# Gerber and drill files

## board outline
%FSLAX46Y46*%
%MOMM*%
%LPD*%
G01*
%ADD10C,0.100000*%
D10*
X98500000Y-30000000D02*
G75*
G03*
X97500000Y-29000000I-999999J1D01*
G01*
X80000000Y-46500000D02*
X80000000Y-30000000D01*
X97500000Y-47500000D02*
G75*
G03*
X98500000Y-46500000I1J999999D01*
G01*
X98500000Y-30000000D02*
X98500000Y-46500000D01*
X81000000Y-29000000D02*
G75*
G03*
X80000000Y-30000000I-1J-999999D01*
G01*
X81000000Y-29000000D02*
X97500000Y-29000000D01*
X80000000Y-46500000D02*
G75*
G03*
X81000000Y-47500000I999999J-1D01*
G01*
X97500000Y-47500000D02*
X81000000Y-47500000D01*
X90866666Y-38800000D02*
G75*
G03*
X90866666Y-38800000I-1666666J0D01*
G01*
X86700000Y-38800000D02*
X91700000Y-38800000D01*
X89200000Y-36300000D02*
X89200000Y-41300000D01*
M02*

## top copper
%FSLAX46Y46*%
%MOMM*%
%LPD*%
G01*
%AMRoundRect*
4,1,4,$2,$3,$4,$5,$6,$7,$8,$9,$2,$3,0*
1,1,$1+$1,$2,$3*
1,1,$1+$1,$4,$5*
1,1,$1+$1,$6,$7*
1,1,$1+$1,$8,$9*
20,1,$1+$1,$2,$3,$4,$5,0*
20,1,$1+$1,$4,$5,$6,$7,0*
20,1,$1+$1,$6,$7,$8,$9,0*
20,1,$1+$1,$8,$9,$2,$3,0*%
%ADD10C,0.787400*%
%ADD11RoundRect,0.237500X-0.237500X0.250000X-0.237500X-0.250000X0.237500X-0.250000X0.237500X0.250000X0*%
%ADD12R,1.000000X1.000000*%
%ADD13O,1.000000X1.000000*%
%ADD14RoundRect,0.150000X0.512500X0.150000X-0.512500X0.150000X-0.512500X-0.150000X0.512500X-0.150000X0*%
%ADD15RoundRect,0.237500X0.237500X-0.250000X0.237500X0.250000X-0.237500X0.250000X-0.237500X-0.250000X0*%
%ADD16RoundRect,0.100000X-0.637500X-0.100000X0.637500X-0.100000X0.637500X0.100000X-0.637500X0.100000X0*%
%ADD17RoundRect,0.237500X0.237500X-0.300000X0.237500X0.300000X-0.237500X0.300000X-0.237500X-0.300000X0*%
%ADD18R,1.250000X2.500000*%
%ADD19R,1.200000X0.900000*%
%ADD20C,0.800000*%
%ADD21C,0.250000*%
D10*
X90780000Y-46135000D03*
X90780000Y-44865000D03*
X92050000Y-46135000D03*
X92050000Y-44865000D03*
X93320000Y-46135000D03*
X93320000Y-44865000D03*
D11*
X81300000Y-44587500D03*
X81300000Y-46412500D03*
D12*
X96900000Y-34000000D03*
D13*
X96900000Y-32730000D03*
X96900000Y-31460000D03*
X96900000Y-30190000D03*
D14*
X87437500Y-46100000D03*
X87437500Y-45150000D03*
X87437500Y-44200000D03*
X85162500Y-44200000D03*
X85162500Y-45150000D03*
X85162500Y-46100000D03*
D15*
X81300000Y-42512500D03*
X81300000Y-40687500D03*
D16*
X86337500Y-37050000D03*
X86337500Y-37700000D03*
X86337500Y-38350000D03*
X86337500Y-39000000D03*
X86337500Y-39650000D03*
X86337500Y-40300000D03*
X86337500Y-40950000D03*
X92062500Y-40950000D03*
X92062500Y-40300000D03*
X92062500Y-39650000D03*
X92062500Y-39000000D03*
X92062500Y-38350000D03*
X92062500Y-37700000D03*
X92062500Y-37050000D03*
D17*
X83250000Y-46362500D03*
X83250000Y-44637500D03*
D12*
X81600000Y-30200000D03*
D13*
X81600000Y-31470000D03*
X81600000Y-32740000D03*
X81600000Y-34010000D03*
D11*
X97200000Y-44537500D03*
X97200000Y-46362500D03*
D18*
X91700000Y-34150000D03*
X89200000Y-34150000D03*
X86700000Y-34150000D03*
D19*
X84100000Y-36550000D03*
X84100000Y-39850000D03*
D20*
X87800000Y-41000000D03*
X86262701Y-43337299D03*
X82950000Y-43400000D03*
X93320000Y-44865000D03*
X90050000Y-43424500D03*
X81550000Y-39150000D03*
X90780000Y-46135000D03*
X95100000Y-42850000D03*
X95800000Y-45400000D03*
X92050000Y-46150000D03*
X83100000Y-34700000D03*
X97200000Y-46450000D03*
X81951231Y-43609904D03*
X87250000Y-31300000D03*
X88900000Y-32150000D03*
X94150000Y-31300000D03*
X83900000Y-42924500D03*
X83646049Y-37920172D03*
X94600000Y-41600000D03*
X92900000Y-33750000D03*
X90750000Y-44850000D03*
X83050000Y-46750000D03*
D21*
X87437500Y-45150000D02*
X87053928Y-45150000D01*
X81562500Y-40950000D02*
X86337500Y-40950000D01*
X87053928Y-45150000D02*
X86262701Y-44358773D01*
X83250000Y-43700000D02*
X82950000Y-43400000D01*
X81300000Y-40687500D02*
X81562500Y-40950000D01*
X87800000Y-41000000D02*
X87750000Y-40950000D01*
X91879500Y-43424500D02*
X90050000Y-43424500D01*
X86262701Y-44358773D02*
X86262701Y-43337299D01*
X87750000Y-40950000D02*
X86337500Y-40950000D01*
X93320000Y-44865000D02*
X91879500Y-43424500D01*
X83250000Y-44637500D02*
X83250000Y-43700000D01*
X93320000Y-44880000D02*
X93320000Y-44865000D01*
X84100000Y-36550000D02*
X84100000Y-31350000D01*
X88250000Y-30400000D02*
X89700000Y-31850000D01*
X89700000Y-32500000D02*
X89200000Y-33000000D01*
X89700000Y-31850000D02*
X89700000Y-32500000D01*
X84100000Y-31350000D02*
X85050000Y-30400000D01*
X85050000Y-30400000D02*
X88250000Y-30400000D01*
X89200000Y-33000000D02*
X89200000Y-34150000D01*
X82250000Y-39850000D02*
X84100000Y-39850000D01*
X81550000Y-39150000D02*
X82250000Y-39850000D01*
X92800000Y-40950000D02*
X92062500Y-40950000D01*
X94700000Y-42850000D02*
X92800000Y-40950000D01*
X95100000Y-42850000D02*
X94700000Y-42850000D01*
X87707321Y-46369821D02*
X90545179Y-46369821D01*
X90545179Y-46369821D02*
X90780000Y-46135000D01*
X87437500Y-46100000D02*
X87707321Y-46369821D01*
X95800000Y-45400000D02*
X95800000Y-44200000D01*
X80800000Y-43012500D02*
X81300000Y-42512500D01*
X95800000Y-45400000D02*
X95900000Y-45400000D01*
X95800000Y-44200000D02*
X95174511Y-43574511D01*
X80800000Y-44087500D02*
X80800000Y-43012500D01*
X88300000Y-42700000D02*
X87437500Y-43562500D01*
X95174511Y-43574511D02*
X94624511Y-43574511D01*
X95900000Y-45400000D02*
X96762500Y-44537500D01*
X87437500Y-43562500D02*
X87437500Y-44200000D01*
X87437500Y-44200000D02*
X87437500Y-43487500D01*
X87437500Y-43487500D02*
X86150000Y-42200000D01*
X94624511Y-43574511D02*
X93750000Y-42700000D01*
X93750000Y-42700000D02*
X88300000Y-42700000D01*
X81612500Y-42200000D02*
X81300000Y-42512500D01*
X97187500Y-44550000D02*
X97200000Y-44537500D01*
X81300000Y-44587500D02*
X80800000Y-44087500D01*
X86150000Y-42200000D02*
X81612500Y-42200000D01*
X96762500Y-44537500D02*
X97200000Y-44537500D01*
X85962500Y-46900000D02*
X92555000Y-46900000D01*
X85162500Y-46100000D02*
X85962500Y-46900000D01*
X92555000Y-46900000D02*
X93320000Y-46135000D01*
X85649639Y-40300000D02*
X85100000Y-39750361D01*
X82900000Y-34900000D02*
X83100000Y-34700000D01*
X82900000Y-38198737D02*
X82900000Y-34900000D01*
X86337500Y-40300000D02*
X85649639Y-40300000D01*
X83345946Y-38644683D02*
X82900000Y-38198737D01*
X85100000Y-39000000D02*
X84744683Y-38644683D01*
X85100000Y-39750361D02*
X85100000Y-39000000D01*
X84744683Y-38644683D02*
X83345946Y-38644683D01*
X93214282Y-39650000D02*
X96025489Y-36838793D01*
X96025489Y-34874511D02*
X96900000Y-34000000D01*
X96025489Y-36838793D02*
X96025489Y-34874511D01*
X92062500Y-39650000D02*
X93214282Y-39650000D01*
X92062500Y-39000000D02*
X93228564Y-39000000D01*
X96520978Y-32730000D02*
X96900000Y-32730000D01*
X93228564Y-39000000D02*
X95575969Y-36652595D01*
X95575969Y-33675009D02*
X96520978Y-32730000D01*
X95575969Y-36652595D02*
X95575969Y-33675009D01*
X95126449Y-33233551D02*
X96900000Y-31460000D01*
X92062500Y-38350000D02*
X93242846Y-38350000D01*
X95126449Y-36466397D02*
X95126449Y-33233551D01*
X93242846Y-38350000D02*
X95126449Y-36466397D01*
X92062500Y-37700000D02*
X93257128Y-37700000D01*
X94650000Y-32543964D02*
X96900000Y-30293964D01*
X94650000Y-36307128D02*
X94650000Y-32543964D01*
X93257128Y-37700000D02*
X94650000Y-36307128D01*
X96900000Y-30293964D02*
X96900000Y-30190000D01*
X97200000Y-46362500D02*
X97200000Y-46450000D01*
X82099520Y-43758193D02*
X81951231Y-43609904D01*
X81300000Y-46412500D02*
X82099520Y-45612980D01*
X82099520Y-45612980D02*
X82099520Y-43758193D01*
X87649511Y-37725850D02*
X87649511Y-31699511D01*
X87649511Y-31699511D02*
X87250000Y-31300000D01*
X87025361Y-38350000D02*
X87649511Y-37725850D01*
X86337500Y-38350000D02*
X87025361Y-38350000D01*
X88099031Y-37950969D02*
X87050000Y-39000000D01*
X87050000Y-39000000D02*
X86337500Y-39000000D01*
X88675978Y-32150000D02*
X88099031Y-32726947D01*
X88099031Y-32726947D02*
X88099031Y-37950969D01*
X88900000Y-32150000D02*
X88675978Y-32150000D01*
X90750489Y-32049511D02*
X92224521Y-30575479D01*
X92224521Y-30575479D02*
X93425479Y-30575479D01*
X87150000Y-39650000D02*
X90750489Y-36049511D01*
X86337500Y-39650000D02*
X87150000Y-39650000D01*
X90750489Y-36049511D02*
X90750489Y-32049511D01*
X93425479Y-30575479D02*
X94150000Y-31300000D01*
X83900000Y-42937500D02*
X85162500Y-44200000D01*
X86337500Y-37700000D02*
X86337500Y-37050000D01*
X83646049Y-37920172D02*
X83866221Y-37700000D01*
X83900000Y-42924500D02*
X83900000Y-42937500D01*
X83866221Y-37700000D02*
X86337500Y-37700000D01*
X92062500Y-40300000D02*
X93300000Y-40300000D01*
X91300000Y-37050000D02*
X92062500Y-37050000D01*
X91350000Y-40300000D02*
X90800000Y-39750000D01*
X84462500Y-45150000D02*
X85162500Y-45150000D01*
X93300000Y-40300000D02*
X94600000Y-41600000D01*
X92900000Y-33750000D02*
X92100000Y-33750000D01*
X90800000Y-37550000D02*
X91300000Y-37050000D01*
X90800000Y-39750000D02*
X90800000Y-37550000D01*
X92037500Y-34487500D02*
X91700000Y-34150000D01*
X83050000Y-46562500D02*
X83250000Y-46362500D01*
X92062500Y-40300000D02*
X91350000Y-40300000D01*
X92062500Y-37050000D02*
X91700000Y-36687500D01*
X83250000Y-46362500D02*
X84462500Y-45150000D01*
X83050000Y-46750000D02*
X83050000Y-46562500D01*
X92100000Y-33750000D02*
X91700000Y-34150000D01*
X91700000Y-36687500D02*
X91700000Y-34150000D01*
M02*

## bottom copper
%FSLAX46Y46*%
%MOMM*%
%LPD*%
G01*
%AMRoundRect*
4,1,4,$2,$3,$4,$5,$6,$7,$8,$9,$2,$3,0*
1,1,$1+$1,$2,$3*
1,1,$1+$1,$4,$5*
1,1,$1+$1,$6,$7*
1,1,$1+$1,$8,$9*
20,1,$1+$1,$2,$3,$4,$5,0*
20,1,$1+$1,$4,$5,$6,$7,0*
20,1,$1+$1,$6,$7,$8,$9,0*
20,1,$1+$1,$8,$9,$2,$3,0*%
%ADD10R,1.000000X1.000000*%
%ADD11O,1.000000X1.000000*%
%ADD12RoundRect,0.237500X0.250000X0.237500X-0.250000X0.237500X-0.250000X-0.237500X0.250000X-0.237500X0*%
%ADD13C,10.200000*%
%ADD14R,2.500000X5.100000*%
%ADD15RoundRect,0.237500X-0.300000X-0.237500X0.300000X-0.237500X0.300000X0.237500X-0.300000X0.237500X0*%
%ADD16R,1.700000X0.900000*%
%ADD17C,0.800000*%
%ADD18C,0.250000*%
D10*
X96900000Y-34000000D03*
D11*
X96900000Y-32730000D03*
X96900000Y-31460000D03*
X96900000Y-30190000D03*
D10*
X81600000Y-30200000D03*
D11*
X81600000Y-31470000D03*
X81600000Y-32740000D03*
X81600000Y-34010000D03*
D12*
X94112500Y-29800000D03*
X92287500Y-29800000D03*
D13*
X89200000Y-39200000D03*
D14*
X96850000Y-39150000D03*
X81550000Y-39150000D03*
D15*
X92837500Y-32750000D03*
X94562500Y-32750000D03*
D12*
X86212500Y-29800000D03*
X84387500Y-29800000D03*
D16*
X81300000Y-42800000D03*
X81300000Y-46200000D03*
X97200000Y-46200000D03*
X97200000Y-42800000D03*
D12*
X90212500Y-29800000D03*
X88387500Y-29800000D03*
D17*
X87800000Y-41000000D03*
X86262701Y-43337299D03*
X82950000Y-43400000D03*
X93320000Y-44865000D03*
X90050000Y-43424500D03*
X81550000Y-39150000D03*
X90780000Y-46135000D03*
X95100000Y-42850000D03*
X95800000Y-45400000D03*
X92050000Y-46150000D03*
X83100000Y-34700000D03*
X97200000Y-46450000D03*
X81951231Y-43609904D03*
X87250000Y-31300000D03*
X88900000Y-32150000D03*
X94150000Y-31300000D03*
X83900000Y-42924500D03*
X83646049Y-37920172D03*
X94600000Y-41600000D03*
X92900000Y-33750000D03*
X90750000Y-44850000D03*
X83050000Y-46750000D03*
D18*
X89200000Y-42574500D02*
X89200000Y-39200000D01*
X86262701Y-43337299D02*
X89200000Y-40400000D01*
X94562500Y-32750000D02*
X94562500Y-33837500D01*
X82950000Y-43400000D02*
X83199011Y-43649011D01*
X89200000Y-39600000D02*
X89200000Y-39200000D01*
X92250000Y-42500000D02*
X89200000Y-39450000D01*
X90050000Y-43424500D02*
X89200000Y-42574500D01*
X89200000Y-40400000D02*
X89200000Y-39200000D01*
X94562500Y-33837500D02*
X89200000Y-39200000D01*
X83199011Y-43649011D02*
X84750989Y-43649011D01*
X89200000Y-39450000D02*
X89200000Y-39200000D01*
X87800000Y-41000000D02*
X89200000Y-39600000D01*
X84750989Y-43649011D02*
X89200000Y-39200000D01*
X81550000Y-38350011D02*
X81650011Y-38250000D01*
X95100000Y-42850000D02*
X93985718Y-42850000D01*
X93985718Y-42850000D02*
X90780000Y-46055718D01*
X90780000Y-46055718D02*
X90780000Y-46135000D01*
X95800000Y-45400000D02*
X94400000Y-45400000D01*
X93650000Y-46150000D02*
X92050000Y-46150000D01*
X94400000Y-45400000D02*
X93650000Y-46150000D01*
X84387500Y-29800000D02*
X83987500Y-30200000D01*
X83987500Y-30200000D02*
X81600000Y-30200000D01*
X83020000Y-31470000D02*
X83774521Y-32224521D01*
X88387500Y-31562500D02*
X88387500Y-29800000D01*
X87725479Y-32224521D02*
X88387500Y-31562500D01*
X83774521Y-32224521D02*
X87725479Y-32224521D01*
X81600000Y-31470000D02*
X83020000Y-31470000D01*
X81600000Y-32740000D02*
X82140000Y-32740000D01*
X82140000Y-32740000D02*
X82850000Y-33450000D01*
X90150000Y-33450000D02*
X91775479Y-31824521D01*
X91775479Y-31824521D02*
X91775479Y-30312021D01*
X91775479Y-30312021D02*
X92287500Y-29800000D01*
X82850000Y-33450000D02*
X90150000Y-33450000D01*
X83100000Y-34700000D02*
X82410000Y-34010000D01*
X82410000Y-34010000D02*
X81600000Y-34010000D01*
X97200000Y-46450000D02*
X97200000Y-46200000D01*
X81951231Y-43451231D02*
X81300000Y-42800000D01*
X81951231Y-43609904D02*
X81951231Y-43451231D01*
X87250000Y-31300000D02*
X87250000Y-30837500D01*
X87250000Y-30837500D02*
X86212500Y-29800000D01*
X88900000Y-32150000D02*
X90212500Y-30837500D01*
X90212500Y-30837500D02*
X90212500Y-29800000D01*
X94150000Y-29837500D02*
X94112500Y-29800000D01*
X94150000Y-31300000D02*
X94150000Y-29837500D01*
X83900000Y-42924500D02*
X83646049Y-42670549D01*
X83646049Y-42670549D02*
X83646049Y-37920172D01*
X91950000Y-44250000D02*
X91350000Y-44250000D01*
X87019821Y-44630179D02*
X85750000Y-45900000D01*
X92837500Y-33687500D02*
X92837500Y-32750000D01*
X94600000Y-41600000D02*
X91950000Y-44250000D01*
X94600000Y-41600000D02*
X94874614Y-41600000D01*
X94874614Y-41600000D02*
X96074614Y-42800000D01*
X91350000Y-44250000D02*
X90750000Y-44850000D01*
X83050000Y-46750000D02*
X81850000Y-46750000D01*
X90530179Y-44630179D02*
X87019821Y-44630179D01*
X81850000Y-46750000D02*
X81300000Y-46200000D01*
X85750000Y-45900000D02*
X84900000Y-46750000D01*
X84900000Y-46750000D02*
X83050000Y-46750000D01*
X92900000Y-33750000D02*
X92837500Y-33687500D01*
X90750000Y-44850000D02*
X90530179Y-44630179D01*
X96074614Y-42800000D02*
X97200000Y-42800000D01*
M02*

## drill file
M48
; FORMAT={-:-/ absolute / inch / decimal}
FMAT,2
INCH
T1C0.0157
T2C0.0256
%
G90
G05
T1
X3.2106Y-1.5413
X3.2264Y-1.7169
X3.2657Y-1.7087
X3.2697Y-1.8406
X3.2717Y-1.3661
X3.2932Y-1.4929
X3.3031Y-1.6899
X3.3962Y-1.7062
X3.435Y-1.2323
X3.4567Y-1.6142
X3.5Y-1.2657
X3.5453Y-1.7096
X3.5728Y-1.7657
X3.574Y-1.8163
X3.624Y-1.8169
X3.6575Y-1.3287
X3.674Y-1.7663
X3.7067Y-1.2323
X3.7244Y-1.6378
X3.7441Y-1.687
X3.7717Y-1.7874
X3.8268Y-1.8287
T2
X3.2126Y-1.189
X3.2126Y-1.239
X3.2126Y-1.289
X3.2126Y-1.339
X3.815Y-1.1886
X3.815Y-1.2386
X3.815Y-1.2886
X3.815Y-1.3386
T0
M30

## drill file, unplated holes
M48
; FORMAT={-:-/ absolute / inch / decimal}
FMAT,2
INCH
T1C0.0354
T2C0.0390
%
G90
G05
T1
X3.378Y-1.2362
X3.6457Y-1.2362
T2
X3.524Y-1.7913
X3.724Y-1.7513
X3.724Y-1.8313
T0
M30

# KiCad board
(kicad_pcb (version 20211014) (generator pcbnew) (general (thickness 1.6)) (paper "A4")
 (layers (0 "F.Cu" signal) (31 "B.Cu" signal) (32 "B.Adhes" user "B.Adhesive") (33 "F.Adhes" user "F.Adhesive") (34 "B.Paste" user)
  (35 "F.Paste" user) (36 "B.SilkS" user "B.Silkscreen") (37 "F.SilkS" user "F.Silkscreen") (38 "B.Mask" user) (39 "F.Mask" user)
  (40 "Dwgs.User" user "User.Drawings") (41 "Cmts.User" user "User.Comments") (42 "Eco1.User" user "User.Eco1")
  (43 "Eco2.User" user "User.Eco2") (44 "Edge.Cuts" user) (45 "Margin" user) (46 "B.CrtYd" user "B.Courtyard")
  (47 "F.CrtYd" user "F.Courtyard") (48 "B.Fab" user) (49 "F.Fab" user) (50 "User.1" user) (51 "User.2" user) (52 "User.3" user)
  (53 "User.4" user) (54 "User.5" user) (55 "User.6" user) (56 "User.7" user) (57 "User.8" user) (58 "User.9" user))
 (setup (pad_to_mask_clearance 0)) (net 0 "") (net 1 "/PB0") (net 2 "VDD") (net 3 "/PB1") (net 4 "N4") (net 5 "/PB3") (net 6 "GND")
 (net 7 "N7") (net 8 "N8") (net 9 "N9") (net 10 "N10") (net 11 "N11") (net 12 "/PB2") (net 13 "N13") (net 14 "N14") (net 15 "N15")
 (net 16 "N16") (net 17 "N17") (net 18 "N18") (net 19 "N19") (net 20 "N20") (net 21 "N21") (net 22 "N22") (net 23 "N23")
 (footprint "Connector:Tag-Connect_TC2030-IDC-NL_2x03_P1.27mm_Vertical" (layer "F.Cu") (at 92.05 45.5)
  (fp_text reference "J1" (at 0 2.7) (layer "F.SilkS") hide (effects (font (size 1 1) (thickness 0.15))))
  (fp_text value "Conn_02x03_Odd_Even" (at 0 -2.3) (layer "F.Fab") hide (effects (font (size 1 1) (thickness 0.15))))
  (pad "" np_thru_hole circle locked (at 2.54 -1.016) (size 0.9906 0.9906) (drill 0.9906) (layers *.Cu *.Mask))
  (pad "" np_thru_hole circle locked (at -2.54 0) (size 0.9906 0.9906) (drill 0.9906) (layers *.Cu *.Mask))
  (pad "" np_thru_hole circle locked (at 2.54 1.016) (size 0.9906 0.9906) (drill 0.9906) (layers *.Cu *.Mask))
  (pad "1" connect circle locked (at -1.27 0.635) (size 0.7874 0.7874) (layers "F.Cu" "F.Mask") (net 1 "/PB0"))
  (pad "2" connect circle locked (at -1.27 -0.635) (size 0.7874 0.7874) (layers "F.Cu" "F.Mask") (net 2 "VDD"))
  (pad "3" connect circle locked (at 0 0.635) (size 0.7874 0.7874) (layers "F.Cu" "F.Mask") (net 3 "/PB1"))
  (pad "4" connect circle locked (at 0 -0.635) (size 0.7874 0.7874) (layers "F.Cu" "F.Mask") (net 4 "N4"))
  (pad "5" connect circle locked (at 1.27 0.635) (size 0.7874 0.7874) (layers "F.Cu" "F.Mask") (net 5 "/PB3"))
  (pad "6" connect circle locked (at 1.27 -0.635) (size 0.7874 0.7874) (layers "F.Cu" "F.Mask") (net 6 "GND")))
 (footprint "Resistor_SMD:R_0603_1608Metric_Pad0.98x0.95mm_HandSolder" (layer "F.Cu") (at 81.3 45.5 -90)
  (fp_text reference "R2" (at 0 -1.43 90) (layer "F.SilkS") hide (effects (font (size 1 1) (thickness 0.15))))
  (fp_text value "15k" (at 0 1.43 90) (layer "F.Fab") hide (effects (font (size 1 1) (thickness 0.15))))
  (pad "1" smd roundrect locked (at -0.9125 0 270) (size 0.975 0.95) (layers "F.Cu" "F.Paste" "F.Mask") (roundrect_rratio 0.25)
   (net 3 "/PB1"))
  (pad "2" smd roundrect locked (at 0.9125 0 270) (size 0.975 0.95) (layers "F.Cu" "F.Paste" "F.Mask") (roundrect_rratio 0.25) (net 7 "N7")))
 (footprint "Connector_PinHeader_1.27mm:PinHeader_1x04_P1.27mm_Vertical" (layer "F.Cu") (at 96.9 34 180)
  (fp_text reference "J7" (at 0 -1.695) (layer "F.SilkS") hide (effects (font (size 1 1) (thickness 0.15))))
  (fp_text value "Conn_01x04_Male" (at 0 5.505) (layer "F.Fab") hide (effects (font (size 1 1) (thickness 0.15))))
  (pad "1" thru_hole rect locked (at 0 0 180) (size 1 1) (drill 0.65) (layers *.Cu *.Mask) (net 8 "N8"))
  (pad "2" thru_hole oval locked (at 0 1.27 180) (size 1 1) (drill 0.65) (layers *.Cu *.Mask) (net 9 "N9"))
  (pad "3" thru_hole oval locked (at 0 2.54 180) (size 1 1) (drill 0.65) (layers *.Cu *.Mask) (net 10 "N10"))
  (pad "4" thru_hole oval locked (at 0 3.81 180) (size 1 1) (drill 0.65) (layers *.Cu *.Mask) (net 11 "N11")))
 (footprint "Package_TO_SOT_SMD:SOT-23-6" (layer "F.Cu") (at 86.3 45.15 180)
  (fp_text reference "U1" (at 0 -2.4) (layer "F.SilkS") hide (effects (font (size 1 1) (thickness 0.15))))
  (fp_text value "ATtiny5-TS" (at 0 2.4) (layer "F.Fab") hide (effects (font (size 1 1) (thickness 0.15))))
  (pad "1" smd roundrect locked (at -1.1375 -0.95 180) (size 1.325 0.6) (layers "F.Cu" "F.Paste" "F.Mask") (roundrect_rratio 0.25)
   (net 1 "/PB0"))
  (pad "2" smd roundrect locked (at -1.1375 0 180) (size 1.325 0.6) (layers "F.Cu" "F.Paste" "F.Mask") (roundrect_rratio 0.25) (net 6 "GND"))
  (pad "3" smd roundrect locked (at -1.1375 0.95 180) (size 1.325 0.6) (layers "F.Cu" "F.Paste" "F.Mask") (roundrect_rratio 0.25)
   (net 3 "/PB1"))
  (pad "4" smd roundrect locked (at 1.1375 0.95 180) (size 1.325 0.6) (layers "F.Cu" "F.Paste" "F.Mask") (roundrect_rratio 0.25)
   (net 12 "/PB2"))
  (pad "5" smd roundrect locked (at 1.1375 0 180) (size 1.325 0.6) (layers "F.Cu" "F.Paste" "F.Mask") (roundrect_rratio 0.25) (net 2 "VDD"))
  (pad "6" smd roundrect locked (at 1.1375 -0.95 180) (size 1.325 0.6) (layers "F.Cu" "F.Paste" "F.Mask") (roundrect_rratio 0.25)
   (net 5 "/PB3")))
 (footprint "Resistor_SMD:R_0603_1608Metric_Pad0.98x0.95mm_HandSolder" (layer "F.Cu") (at 81.3 41.6 90)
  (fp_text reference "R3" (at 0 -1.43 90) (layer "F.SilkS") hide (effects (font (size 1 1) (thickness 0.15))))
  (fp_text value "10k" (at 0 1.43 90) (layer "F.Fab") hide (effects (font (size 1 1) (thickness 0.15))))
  (pad "1" smd roundrect locked (at -0.9125 0 90) (size 0.975 0.95) (layers "F.Cu" "F.Paste" "F.Mask") (roundrect_rratio 0.25)
   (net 3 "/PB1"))
  (pad "2" smd roundrect locked (at 0.9125 0 90) (size 0.975 0.95) (layers "F.Cu" "F.Paste" "F.Mask") (roundrect_rratio 0.25) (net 6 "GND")))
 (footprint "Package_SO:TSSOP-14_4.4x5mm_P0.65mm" (layer "F.Cu") (at 89.2 39)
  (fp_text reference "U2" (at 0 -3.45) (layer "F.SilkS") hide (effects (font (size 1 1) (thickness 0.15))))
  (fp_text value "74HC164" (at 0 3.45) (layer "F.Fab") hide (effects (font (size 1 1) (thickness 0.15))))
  (pad "1" smd roundrect locked (at -2.8625 -1.95) (size 1.475 0.4) (layers "F.Cu" "F.Paste" "F.Mask") (roundrect_rratio 0.25)
   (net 12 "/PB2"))
  (pad "2" smd roundrect locked (at -2.8625 -1.3) (size 1.475 0.4) (layers "F.Cu" "F.Paste" "F.Mask") (roundrect_rratio 0.25)
   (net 12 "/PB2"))
  (pad "3" smd roundrect locked (at -2.8625 -0.65) (size 1.475 0.4) (layers "F.Cu" "F.Paste" "F.Mask") (roundrect_rratio 0.25)
   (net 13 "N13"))
  (pad "4" smd roundrect locked (at -2.8625 0) (size 1.475 0.4) (layers "F.Cu" "F.Paste" "F.Mask") (roundrect_rratio 0.25) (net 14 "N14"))
  (pad "5" smd roundrect locked (at -2.8625 0.65) (size 1.475 0.4) (layers "F.Cu" "F.Paste" "F.Mask") (roundrect_rratio 0.25) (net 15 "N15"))
  (pad "6" smd roundrect locked (at -2.8625 1.3) (size 1.475 0.4) (layers "F.Cu" "F.Paste" "F.Mask") (roundrect_rratio 0.25) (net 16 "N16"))
  (pad "7" smd roundrect locked (at -2.8625 1.95) (size 1.475 0.4) (layers "F.Cu" "F.Paste" "F.Mask") (roundrect_rratio 0.25) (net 6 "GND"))
  (pad "8" smd roundrect locked (at 2.8625 1.95) (size 1.475 0.4) (layers "F.Cu" "F.Paste" "F.Mask") (roundrect_rratio 0.25) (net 1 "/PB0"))
  (pad "9" smd roundrect locked (at 2.8625 1.3) (size 1.475 0.4) (layers "F.Cu" "F.Paste" "F.Mask") (roundrect_rratio 0.25) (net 2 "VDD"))
  (pad "10" smd roundrect locked (at 2.8625 0.65) (size 1.475 0.4) (layers "F.Cu" "F.Paste" "F.Mask") (roundrect_rratio 0.25) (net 8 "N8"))
  (pad "11" smd roundrect locked (at 2.8625 0) (size 1.475 0.4) (layers "F.Cu" "F.Paste" "F.Mask") (roundrect_rratio 0.25) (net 9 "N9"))
  (pad "12" smd roundrect locked (at 2.8625 -0.65) (size 1.475 0.4) (layers "F.Cu" "F.Paste" "F.Mask") (roundrect_rratio 0.25)
   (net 10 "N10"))
  (pad "13" smd roundrect locked (at 2.8625 -1.3) (size 1.475 0.4) (layers "F.Cu" "F.Paste" "F.Mask") (roundrect_rratio 0.25) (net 11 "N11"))
  (pad "14" smd roundrect locked (at 2.8625 -1.95) (size 1.475 0.4) (layers "F.Cu" "F.Paste" "F.Mask") (roundrect_rratio 0.25) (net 2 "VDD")))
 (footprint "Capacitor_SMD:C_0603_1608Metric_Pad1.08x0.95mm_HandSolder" (layer "F.Cu") (at 83.25 45.5 90)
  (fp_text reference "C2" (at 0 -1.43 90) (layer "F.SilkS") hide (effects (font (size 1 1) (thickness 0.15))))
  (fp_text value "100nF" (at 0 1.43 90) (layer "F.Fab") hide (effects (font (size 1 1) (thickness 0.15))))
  (pad "1" smd roundrect locked (at -0.8625 0 90) (size 1.075 0.95) (layers "F.Cu" "F.Paste" "F.Mask") (roundrect_rratio 0.25) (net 2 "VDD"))
  (pad "2" smd roundrect locked (at 0.8625 0 90) (size 1.075 0.95) (layers "F.Cu" "F.Paste" "F.Mask") (roundrect_rratio 0.25) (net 6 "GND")))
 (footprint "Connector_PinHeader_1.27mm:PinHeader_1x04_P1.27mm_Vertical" (layer "F.Cu") (at 81.6 30.2)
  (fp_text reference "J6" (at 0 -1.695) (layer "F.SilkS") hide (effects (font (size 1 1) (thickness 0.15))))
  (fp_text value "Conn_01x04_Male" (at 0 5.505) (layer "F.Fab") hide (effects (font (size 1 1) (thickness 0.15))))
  (pad "1" thru_hole rect locked (at 0 0) (size 1 1) (drill 0.65) (layers *.Cu *.Mask) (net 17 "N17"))
  (pad "2" thru_hole oval locked (at 0 1.27) (size 1 1) (drill 0.65) (layers *.Cu *.Mask) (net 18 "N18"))
  (pad "3" thru_hole oval locked (at 0 2.54) (size 1 1) (drill 0.65) (layers *.Cu *.Mask) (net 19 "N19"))
  (pad "4" thru_hole oval locked (at 0 3.81) (size 1 1) (drill 0.65) (layers *.Cu *.Mask) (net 16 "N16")))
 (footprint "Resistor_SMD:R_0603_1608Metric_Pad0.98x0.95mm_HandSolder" (layer "F.Cu") (at 97.2 45.45 -90)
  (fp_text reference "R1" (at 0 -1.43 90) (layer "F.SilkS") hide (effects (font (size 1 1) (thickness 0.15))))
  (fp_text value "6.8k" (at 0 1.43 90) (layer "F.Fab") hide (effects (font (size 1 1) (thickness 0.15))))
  (pad "1" smd roundrect locked (at -0.9125 0 270) (size 0.975 0.95) (layers "F.Cu" "F.Paste" "F.Mask") (roundrect_rratio 0.25)
   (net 3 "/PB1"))
  (pad "2" smd roundrect locked (at 0.9125 0 270) (size 0.975 0.95) (layers "F.Cu" "F.Paste" "F.Mask") (roundrect_rratio 0.25)
   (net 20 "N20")))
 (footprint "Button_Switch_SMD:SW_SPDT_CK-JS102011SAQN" (layer "F.Cu") (at 89.2 31.4 180)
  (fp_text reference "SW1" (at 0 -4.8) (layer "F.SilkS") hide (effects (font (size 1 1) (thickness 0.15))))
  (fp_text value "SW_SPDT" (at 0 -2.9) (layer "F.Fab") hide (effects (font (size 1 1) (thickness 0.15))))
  (pad "" np_thru_hole circle locked (at -3.4 0 180) (size 0.9 0.9) (drill 0.9) (layers *.Cu *.Mask))
  (pad "" np_thru_hole circle locked (at 3.4 0 180) (size 0.9 0.9) (drill 0.9) (layers *.Cu *.Mask))
  (pad "1" smd rect locked (at -2.5 -2.75 180) (size 1.25 2.5) (layers "F.Cu" "F.Paste" "F.Mask") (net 2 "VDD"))
  (pad "2" smd rect locked (at 0 -2.75 180) (size 1.25 2.5) (layers "F.Cu" "F.Paste" "F.Mask") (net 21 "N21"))
  (pad "3" smd rect locked (at 2.5 -2.75 180) (size 1.25 2.5) (layers "F.Cu" "F.Paste" "F.Mask") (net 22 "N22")))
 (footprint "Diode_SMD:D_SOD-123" (layer "F.Cu") (at 84.1 38.2 -90)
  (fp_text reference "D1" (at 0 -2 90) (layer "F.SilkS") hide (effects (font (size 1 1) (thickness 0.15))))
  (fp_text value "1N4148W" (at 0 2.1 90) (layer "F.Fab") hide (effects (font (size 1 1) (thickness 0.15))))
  (pad "1" smd rect locked (at -1.65 0 270) (size 0.9 1.2) (layers "F.Cu" "F.Paste" "F.Mask") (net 21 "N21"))
  (pad "2" smd rect locked (at 1.65 0 270) (size 0.9 1.2) (layers "F.Cu" "F.Paste" "F.Mask") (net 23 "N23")))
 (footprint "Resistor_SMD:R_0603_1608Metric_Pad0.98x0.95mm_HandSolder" (layer "B.Cu") (at 93.2 29.8 180)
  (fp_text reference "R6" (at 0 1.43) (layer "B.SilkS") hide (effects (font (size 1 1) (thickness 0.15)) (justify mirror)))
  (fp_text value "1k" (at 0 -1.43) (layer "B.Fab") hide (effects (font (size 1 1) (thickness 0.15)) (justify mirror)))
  (pad "1" smd roundrect locked (at -0.9125 0 180) (size 0.975 0.95) (layers "B.Cu" "B.Paste" "B.Mask") (roundrect_rratio 0.25)
   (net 15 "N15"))
  (pad "2" smd roundrect locked (at 0.9125 0 180) (size 0.975 0.95) (layers "B.Cu" "B.Paste" "B.Mask") (roundrect_rratio 0.25)
   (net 19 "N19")))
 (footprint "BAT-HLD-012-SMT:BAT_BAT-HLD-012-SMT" (layer "B.Cu") (at 89.2 39.2 180)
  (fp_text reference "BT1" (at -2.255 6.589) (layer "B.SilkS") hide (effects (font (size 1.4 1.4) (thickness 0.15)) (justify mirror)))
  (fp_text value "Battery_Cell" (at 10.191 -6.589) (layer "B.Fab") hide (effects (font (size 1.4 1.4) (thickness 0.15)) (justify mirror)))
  (pad "N" smd circle locked (at 0 0 180) (size 10.2 10.2) (layers "B.Cu" "B.Mask") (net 6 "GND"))
  (pad "P1" smd rect locked (at -7.65 0.05 180) (size 2.5 5.1) (layers "B.Cu" "B.Paste" "B.Mask"))
  (pad "P2" smd rect locked (at 7.65 0.05 180) (size 2.5 5.1) (layers "B.Cu" "B.Paste" "B.Mask") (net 23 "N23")))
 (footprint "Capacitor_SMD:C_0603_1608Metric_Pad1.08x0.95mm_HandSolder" (layer "B.Cu") (at 93.7 32.75)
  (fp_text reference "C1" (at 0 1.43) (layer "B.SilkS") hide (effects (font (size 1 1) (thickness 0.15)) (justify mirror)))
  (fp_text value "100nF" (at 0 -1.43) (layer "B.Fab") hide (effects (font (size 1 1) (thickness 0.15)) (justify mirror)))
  (pad "1" smd roundrect locked (at -0.8625 0) (size 1.075 0.95) (layers "B.Cu" "B.Paste" "B.Mask") (roundrect_rratio 0.25) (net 2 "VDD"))
  (pad "2" smd roundrect locked (at 0.8625 0) (size 1.075 0.95) (layers "B.Cu" "B.Paste" "B.Mask") (roundrect_rratio 0.25) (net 6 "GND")))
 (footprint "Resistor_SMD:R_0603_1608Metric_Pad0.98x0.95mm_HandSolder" (layer "B.Cu") (at 85.3 29.8 180)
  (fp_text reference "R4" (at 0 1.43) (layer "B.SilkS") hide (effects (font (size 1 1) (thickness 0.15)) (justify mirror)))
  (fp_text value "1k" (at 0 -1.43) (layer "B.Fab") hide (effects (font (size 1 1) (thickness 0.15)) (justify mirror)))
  (pad "1" smd roundrect locked (at -0.9125 0 180) (size 0.975 0.95) (layers "B.Cu" "B.Paste" "B.Mask") (roundrect_rratio 0.25)
   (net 13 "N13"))
  (pad "2" smd roundrect locked (at 0.9125 0 180) (size 0.975 0.95) (layers "B.Cu" "B.Paste" "B.Mask") (roundrect_rratio 0.25)
   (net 17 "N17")))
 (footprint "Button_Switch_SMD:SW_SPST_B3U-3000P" (layer "B.Cu") (at 81.3 44.5 -90)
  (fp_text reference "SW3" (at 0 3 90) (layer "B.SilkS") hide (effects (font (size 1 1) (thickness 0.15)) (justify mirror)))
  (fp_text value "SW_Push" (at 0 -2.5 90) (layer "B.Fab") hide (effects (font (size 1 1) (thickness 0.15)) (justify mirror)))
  (pad "1" smd rect locked (at -1.7 0 270) (size 0.9 1.7) (layers "B.Cu" "B.Paste" "B.Mask") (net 7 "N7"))
  (pad "2" smd rect locked (at 1.7 0 270) (size 0.9 1.7) (layers "B.Cu" "B.Paste" "B.Mask") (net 2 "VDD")))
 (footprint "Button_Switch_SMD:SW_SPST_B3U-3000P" (layer "B.Cu") (at 97.2 44.5 90)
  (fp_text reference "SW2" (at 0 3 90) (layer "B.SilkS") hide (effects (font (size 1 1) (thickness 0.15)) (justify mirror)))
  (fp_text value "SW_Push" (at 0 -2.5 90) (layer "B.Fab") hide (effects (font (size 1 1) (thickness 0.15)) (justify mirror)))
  (pad "1" smd rect locked (at -1.7 0 90) (size 0.9 1.7) (layers "B.Cu" "B.Paste" "B.Mask") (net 20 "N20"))
  (pad "2" smd rect locked (at 1.7 0 90) (size 0.9 1.7) (layers "B.Cu" "B.Paste" "B.Mask") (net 2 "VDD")))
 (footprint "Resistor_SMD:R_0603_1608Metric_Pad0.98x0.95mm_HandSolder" (layer "B.Cu") (at 89.3 29.8 180)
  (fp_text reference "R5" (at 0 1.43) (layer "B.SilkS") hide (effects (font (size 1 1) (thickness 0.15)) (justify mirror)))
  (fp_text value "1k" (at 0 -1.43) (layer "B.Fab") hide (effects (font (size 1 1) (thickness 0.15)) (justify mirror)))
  (pad "1" smd roundrect locked (at -0.9125 0 180) (size 0.975 0.95) (layers "B.Cu" "B.Paste" "B.Mask") (roundrect_rratio 0.25)
   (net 14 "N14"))
  (pad "2" smd roundrect locked (at 0.9125 0 180) (size 0.975 0.95) (layers "B.Cu" "B.Paste" "B.Mask") (roundrect_rratio 0.25)
   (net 18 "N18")))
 (gr_arc (start 97.5 29) (mid 98.207107 29.292893) (end 98.5 30) (layer "Edge.Cuts") (width 0.1))
 (gr_line (start 80 46.5) (end 80 30) (layer "Edge.Cuts") (width 0.1))
 (gr_arc (start 98.5 46.5) (mid 98.207107 47.207107) (end 97.5 47.5) (layer "Edge.Cuts") (width 0.1))
 (gr_line (start 98.5 30) (end 98.5 46.5) (layer "Edge.Cuts") (width 0.1))
 (gr_arc (start 80 30) (mid 80.292893 29.292893) (end 81 29) (layer "Edge.Cuts") (width 0.1))
 (gr_line (start 81 29) (end 97.5 29) (layer "Edge.Cuts") (width 0.1))
 (gr_arc (start 81 47.5) (mid 80.292893 47.207107) (end 80 46.5) (layer "Edge.Cuts") (width 0.1))
 (gr_line (start 97.5 47.5) (end 81 47.5) (layer "Edge.Cuts") (width 0.1))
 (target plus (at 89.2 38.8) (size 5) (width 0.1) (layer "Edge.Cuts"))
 (segment (start 87.4375 45.15) (end 87.053928 45.15) (width 0.25) (layer "F.Cu") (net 6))
 (segment (start 81.5625 40.95) (end 86.3375 40.95) (width 0.25) (layer "F.Cu") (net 6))
 (segment (start 87.053928 45.15) (end 86.262701 44.358773) (width 0.25) (layer "F.Cu") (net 6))
 (segment (start 83.25 43.7) (end 82.95 43.4) (width 0.25) (layer "F.Cu") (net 6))
 (segment (start 81.3 40.6875) (end 81.5625 40.95) (width 0.25) (layer "F.Cu") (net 6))
 (segment (start 87.8 41) (end 87.75 40.95) (width 0.25) (layer "F.Cu") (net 6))
 (segment (start 91.8795 43.4245) (end 90.05 43.4245) (width 0.25) (layer "F.Cu") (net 6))
 (segment (start 86.262701 44.358773) (end 86.262701 43.337299) (width 0.25) (layer "F.Cu") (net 6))
 (segment (start 87.75 40.95) (end 86.3375 40.95) (width 0.25) (layer "F.Cu") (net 6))
 (segment (start 93.32 44.865) (end 91.8795 43.4245) (width 0.25) (layer "F.Cu") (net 6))
 (segment (start 83.25 44.6375) (end 83.25 43.7) (width 0.25) (layer "F.Cu") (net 6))
 (segment (start 93.32 44.88) (end 93.32 44.865) (width 0.25) (layer "F.Cu") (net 6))
 (via (at 87.8 41) (size 0.8) (drill 0.4) (layers "F.Cu" "B.Cu") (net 6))
 (via (at 86.262701 43.337299) (size 0.8) (drill 0.4) (layers "F.Cu" "B.Cu") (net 6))
 (via (at 82.95 43.4) (size 0.8) (drill 0.4) (layers "F.Cu" "B.Cu") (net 6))
 (via (at 93.32 44.865) (size 0.8) (drill 0.4) (layers "F.Cu" "B.Cu") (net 6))
 (via (at 90.05 43.4245) (size 0.8) (drill 0.4) (layers "F.Cu" "B.Cu") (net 6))
 (segment (start 89.2 42.5745) (end 89.2 39.2) (width 0.25) (layer "B.Cu") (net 6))
 (segment (start 86.262701 43.337299) (end 89.2 40.4) (width 0.25) (layer "B.Cu") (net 6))
 (segment (start 94.5625 32.75) (end 94.5625 33.8375) (width 0.25) (layer "B.Cu") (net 6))
 (segment (start 82.95 43.4) (end 83.199011 43.649011) (width 0.25) (layer "B.Cu") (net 6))
 (segment (start 89.2 39.6) (end 89.2 39.2) (width 0.25) (layer "B.Cu") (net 6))
 (segment (start 92.25 42.5) (end 89.2 39.45) (width 0.25) (layer "B.Cu") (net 6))
 (segment (start 90.05 43.4245) (end 89.2 42.5745) (width 0.25) (layer "B.Cu") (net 6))
 (segment (start 89.2 40.4) (end 89.2 39.2) (width 0.25) (layer "B.Cu") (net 6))
 (segment (start 94.5625 33.8375) (end 89.2 39.2) (width 0.25) (layer "B.Cu") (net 6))
 (segment (start 83.199011 43.649011) (end 84.750989 43.649011) (width 0.25) (layer "B.Cu") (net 6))
 (segment (start 89.2 39.45) (end 89.2 39.2) (width 0.25) (layer "B.Cu") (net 6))
 (segment (start 87.8 41) (end 89.2 39.6) (width 0.25) (layer "B.Cu") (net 6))
 (segment (start 84.750989 43.649011) (end 89.2 39.2) (width 0.25) (layer "B.Cu") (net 6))
 (segment (start 84.1 36.55) (end 84.1 31.35) (width 0.25) (layer "F.Cu") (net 21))
 (segment (start 88.25 30.4) (end 89.7 31.85) (width 0.25) (layer "F.Cu") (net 21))
 (segment (start 89.7 32.5) (end 89.2 33) (width 0.25) (layer "F.Cu") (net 21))
 (segment (start 89.7 31.85) (end 89.7 32.5) (width 0.25) (layer "F.Cu") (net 21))
 (segment (start 84.1 31.35) (end 85.05 30.4) (width 0.25) (layer "F.Cu") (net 21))
 (segment (start 85.05 30.4) (end 88.25 30.4) (width 0.25) (layer "F.Cu") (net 21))
 (segment (start 89.2 33) (end 89.2 34.15) (width 0.25) (layer "F.Cu") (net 21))
 (segment (start 82.25 39.85) (end 84.1 39.85) (width 0.25) (layer "F.Cu") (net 23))
 (segment (start 81.55 39.15) (end 82.25 39.85) (width 0.25) (layer "F.Cu") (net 23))
 (via (at 81.55 39.15) (size 0.8) (drill 0.4) (layers "F.Cu" "B.Cu") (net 23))
 (segment (start 81.55 38.350011) (end 81.650011 38.25) (width 0.25) (layer "B.Cu") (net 23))
 (segment (start 92.8 40.95) (end 92.0625 40.95) (width 0.25) (layer "F.Cu") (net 1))
 (segment (start 94.7 42.85) (end 92.8 40.95) (width 0.25) (layer "F.Cu") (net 1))
 (segment (start 95.1 42.85) (end 94.7 42.85) (width 0.25) (layer "F.Cu") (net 1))
 (segment (start 87.707321 46.369821) (end 90.545179 46.369821) (width 0.25) (layer "F.Cu") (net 1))
 (segment (start 90.545179 46.369821) (end 90.78 46.135) (width 0.25) (layer "F.Cu") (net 1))
 (segment (start 87.4375 46.1) (end 87.707321 46.369821) (width 0.25) (layer "F.Cu") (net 1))
 (via (at 90.78 46.135) (size 0.8) (drill 0.4) (layers "F.Cu" "B.Cu") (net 1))
 (via (at 95.1 42.85) (size 0.8) (drill 0.4) (layers "F.Cu" "B.Cu") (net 1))
 (segment (start 95.1 42.85) (end 93.985718 42.85) (width 0.25) (layer "B.Cu") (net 1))
 (segment (start 93.985718 42.85) (end 90.78 46.055718) (width 0.25) (layer "B.Cu") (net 1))
 (segment (start 90.78 46.055718) (end 90.78 46.135) (width 0.25) (layer "B.Cu") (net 1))
 (segment (start 95.8 45.4) (end 95.8 44.2) (width 0.25) (layer "F.Cu") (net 3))
 (segment (start 80.8 43.0125) (end 81.3 42.5125) (width 0.25) (layer "F.Cu") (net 3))
 (segment (start 95.8 45.4) (end 95.9 45.4) (width 0.25) (layer "F.Cu") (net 3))
 (segment (start 95.8 44.2) (end 95.174511 43.574511) (width 0.25) (layer "F.Cu") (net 3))
 (segment (start 80.8 44.0875) (end 80.8 43.0125) (width 0.25) (layer "F.Cu") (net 3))
 (segment (start 88.3 42.7) (end 87.4375 43.5625) (width 0.25) (layer "F.Cu") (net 3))
 (segment (start 95.174511 43.574511) (end 94.624511 43.574511) (width 0.25) (layer "F.Cu") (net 3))
 (segment (start 95.9 45.4) (end 96.7625 44.5375) (width 0.25) (layer "F.Cu") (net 3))
 (segment (start 87.4375 43.5625) (end 87.4375 44.2) (width 0.25) (layer "F.Cu") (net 3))
 (segment (start 87.4375 44.2) (end 87.4375 43.4875) (width 0.25) (layer "F.Cu") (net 3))
 (segment (start 87.4375 43.4875) (end 86.15 42.2) (width 0.25) (layer "F.Cu") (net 3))
 (segment (start 94.624511 43.574511) (end 93.75 42.7) (width 0.25) (layer "F.Cu") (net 3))
 (segment (start 93.75 42.7) (end 88.3 42.7) (width 0.25) (layer "F.Cu") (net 3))
 (segment (start 81.6125 42.2) (end 81.3 42.5125) (width 0.25) (layer "F.Cu") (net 3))
 (segment (start 97.1875 44.55) (end 97.2 44.5375) (width 0.25) (layer "F.Cu") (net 3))
 (segment (start 81.3 44.5875) (end 80.8 44.0875) (width 0.25) (layer "F.Cu") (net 3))
 (segment (start 86.15 42.2) (end 81.6125 42.2) (width 0.25) (layer "F.Cu") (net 3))
 (segment (start 96.7625 44.5375) (end 97.2 44.5375) (width 0.25) (layer "F.Cu") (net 3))
 (via (at 95.8 45.4) (size 0.8) (drill 0.4) (layers "F.Cu" "B.Cu") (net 3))
 (via (at 92.05 46.15) (size 0.8) (drill 0.4) (layers "F.Cu" "B.Cu") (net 3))
 (segment (start 95.8 45.4) (end 94.4 45.4) (width 0.25) (layer "B.Cu") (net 3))
 (segment (start 93.65 46.15) (end 92.05 46.15) (width 0.25) (layer "B.Cu") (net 3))
 (segment (start 94.4 45.4) (end 93.65 46.15) (width 0.25) (layer "B.Cu") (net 3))
 (segment (start 85.9625 46.9) (end 92.555 46.9) (width 0.25) (layer "F.Cu") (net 5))
 (segment (start 85.1625 46.1) (end 85.9625 46.9) (width 0.25) (layer "F.Cu") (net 5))
 (segment (start 92.555 46.9) (end 93.32 46.135) (width 0.25) (layer "F.Cu") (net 5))
 (segment (start 84.3875 29.8) (end 83.9875 30.2) (width 0.25) (layer "B.Cu") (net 17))
 (segment (start 83.9875 30.2) (end 81.6 30.2) (width 0.25) (layer "B.Cu") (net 17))
 (segment (start 83.02 31.47) (end 83.774521 32.224521) (width 0.25) (layer "B.Cu") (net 18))
 (segment (start 88.3875 31.5625) (end 88.3875 29.8) (width 0.25) (layer "B.Cu") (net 18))
 (segment (start 87.725479 32.224521) (end 88.3875 31.5625) (width 0.25) (layer "B.Cu") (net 18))
 (segment (start 83.774521 32.224521) (end 87.725479 32.224521) (width 0.25) (layer "B.Cu") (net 18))
 (segment (start 81.6 31.47) (end 83.02 31.47) (width 0.25) (layer "B.Cu") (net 18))
 (segment (start 81.6 32.74) (end 82.14 32.74) (width 0.25) (layer "B.Cu") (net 19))
 (segment (start 82.14 32.74) (end 82.85 33.45) (width 0.25) (layer "B.Cu") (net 19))
 (segment (start 90.15 33.45) (end 91.775479 31.824521) (width 0.25) (layer "B.Cu") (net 19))
 (segment (start 91.775479 31.824521) (end 91.775479 30.312021) (width 0.25) (layer "B.Cu") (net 19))
 (segment (start 91.775479 30.312021) (end 92.2875 29.8) (width 0.25) (layer "B.Cu") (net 19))
 (segment (start 82.85 33.45) (end 90.15 33.45) (width 0.25) (layer "B.Cu") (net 19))
 (segment (start 85.649639 40.3) (end 85.1 39.750361) (width 0.25) (layer "F.Cu") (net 16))
 (segment (start 82.9 34.9) (end 83.1 34.7) (width 0.25) (layer "F.Cu") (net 16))
 (segment (start 82.9 38.198737) (end 82.9 34.9) (width 0.25) (layer "F.Cu") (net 16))
 (segment (start 86.3375 40.3) (end 85.649639 40.3) (width 0.25) (layer "F.Cu") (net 16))
 (segment (start 83.345946 38.644683) (end 82.9 38.198737) (width 0.25) (layer "F.Cu") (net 16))
 (segment (start 85.1 39) (end 84.744683 38.644683) (width 0.25) (layer "F.Cu") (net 16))
 (segment (start 85.1 39.750361) (end 85.1 39) (width 0.25) (layer "F.Cu") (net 16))
 (segment (start 84.744683 38.644683) (end 83.345946 38.644683) (width 0.25) (layer "F.Cu") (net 16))
 (via (at 83.1 34.7) (size 0.8) (drill 0.4) (layers "F.Cu" "B.Cu") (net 16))
 (segment (start 83.1 34.7) (end 82.41 34.01) (width 0.25) (layer "B.Cu") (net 16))
 (segment (start 82.41 34.01) (end 81.6 34.01) (width 0.25) (layer "B.Cu") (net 16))
 (segment (start 93.214282 39.65) (end 96.025489 36.838793) (width 0.25) (layer "F.Cu") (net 8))
 (segment (start 96.025489 34.874511) (end 96.9 34) (width 0.25) (layer "F.Cu") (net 8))
 (segment (start 96.025489 36.838793) (end 96.025489 34.874511) (width 0.25) (layer "F.Cu") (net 8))
 (segment (start 92.0625 39.65) (end 93.214282 39.65) (width 0.25) (layer "F.Cu") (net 8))
 (segment (start 92.0625 39) (end 93.228564 39) (width 0.25) (layer "F.Cu") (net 9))
 (segment (start 96.520978 32.73) (end 96.9 32.73) (width 0.25) (layer "F.Cu") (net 9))
 (segment (start 93.228564 39) (end 95.575969 36.652595) (width 0.25) (layer "F.Cu") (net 9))
 (segment (start 95.575969 33.675009) (end 96.520978 32.73) (width 0.25) (layer "F.Cu") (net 9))
 (segment (start 95.575969 36.652595) (end 95.575969 33.675009) (width 0.25) (layer "F.Cu") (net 9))
 (segment (start 95.126449 33.233551) (end 96.9 31.46) (width 0.25) (layer "F.Cu") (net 10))
 (segment (start 92.0625 38.35) (end 93.242846 38.35) (width 0.25) (layer "F.Cu") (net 10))
 (segment (start 95.126449 36.466397) (end 95.126449 33.233551) (width 0.25) (layer "F.Cu") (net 10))
 (segment (start 93.242846 38.35) (end 95.126449 36.466397) (width 0.25) (layer "F.Cu") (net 10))
 (segment (start 92.0625 37.7) (end 93.257128 37.7) (width 0.25) (layer "F.Cu") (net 11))
 (segment (start 94.65 32.543964) (end 96.9 30.293964) (width 0.25) (layer "F.Cu") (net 11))
 (segment (start 94.65 36.307128) (end 94.65 32.543964) (width 0.25) (layer "F.Cu") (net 11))
 (segment (start 93.257128 37.7) (end 94.65 36.307128) (width 0.25) (layer "F.Cu") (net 11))
 (segment (start 96.9 30.293964) (end 96.9 30.19) (width 0.25) (layer "F.Cu") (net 11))
 (segment (start 97.2 46.3625) (end 97.2 46.45) (width 0.25) (layer "F.Cu") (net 20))
 (via (at 97.2 46.45) (size 0.8) (drill 0.4) (layers "F.Cu" "B.Cu") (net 20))
 (segment (start 97.2 46.45) (end 97.2 46.2) (width 0.25) (layer "B.Cu") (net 20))
 (segment (start 82.09952 43.758193) (end 81.951231 43.609904) (width 0.25) (layer "F.Cu") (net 7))
 (segment (start 81.3 46.4125) (end 82.09952 45.61298) (width 0.25) (layer "F.Cu") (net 7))
 (segment (start 82.09952 45.61298) (end 82.09952 43.758193) (width 0.25) (layer "F.Cu") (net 7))
 (via (at 81.951231 43.609904) (size 0.8) (drill 0.4) (layers "F.Cu" "B.Cu") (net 7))
 (segment (start 81.951231 43.451231) (end 81.3 42.8) (width 0.25) (layer "B.Cu") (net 7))
 (segment (start 81.951231 43.609904) (end 81.951231 43.451231) (width 0.25) (layer "B.Cu") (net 7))
 (segment (start 87.649511 37.72585) (end 87.649511 31.699511) (width 0.25) (layer "F.Cu") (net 13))
 (segment (start 87.649511 31.699511) (end 87.25 31.3) (width 0.25) (layer "F.Cu") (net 13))
 (segment (start 87.025361 38.35) (end 87.649511 37.72585) (width 0.25) (layer "F.Cu") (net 13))
 (segment (start 86.3375 38.35) (end 87.025361 38.35) (width 0.25) (layer "F.Cu") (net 13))
 (via (at 87.25 31.3) (size 0.8) (drill 0.4) (layers "F.Cu" "B.Cu") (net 13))
 (segment (start 87.25 31.3) (end 87.25 30.8375) (width 0.25) (layer "B.Cu") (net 13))
 (segment (start 87.25 30.8375) (end 86.2125 29.8) (width 0.25) (layer "B.Cu") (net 13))
 (segment (start 88.099031 37.950969) (end 87.05 39) (width 0.25) (layer "F.Cu") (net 14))
 (segment (start 87.05 39) (end 86.3375 39) (width 0.25) (layer "F.Cu") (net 14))
 (segment (start 88.675978 32.15) (end 88.099031 32.726947) (width 0.25) (layer "F.Cu") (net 14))
 (segment (start 88.099031 32.726947) (end 88.099031 37.950969) (width 0.25) (layer "F.Cu") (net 14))
 (segment (start 88.9 32.15) (end 88.675978 32.15) (width 0.25) (layer "F.Cu") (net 14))
 (via (at 88.9 32.15) (size 0.8) (drill 0.4) (layers "F.Cu" "B.Cu") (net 14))
 (segment (start 88.9 32.15) (end 90.2125 30.8375) (width 0.25) (layer "B.Cu") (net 14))
 (segment (start 90.2125 30.8375) (end 90.2125 29.8) (width 0.25) (layer "B.Cu") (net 14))
 (segment (start 90.750489 32.049511) (end 92.224521 30.575479) (width 0.25) (layer "F.Cu") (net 15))
 (segment (start 92.224521 30.575479) (end 93.425479 30.575479) (width 0.25) (layer "F.Cu") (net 15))
 (segment (start 87.15 39.65) (end 90.750489 36.049511) (width 0.25) (layer "F.Cu") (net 15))
 (segment (start 86.3375 39.65) (end 87.15 39.65) (width 0.25) (layer "F.Cu") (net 15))
 (segment (start 90.750489 36.049511) (end 90.750489 32.049511) (width 0.25) (layer "F.Cu") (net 15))
 (segment (start 93.425479 30.575479) (end 94.15 31.3) (width 0.25) (layer "F.Cu") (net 15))
 (via (at 94.15 31.3) (size 0.8) (drill 0.4) (layers "F.Cu" "B.Cu") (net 15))
 (segment (start 94.15 29.8375) (end 94.1125 29.8) (width 0.25) (layer "B.Cu") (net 15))
 (segment (start 94.15 31.3) (end 94.15 29.8375) (width 0.25) (layer "B.Cu") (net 15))
 (segment (start 83.9 42.9375) (end 85.1625 44.2) (width 0.25) (layer "F.Cu") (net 12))
 (segment (start 86.3375 37.7) (end 86.3375 37.05) (width 0.25) (layer "F.Cu") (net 12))
 (segment (start 83.646049 37.920172) (end 83.866221 37.7) (width 0.25) (layer "F.Cu") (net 12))
 (segment (start 83.9 42.9245) (end 83.9 42.9375) (width 0.25) (layer "F.Cu") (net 12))
 (segment (start 83.866221 37.7) (end 86.3375 37.7) (width 0.25) (layer "F.Cu") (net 12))
 (via (at 83.9 42.9245) (size 0.8) (drill 0.4) (layers "F.Cu" "B.Cu") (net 12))
 (via (at 83.646049 37.920172) (size 0.8) (drill 0.4) (layers "F.Cu" "B.Cu") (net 12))
 (segment (start 83.9 42.9245) (end 83.646049 42.670549) (width 0.25) (layer "B.Cu") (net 12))
 (segment (start 83.646049 42.670549) (end 83.646049 37.920172) (width 0.25) (layer "B.Cu") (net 12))
 (segment (start 92.0625 40.3) (end 93.3 40.3) (width 0.25) (layer "F.Cu") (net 2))
 (segment (start 91.3 37.05) (end 92.0625 37.05) (width 0.25) (layer "F.Cu") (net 2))
 (segment (start 91.35 40.3) (end 90.8 39.75) (width 0.25) (layer "F.Cu") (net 2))
 (segment (start 84.4625 45.15) (end 85.1625 45.15) (width 0.25) (layer "F.Cu") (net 2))
 (segment (start 93.3 40.3) (end 94.6 41.6) (width 0.25) (layer "F.Cu") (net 2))
 (segment (start 92.9 33.75) (end 92.1 33.75) (width 0.25) (layer "F.Cu") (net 2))
 (segment (start 90.8 37.55) (end 91.3 37.05) (width 0.25) (layer "F.Cu") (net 2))
 (segment (start 90.8 39.75) (end 90.8 37.55) (width 0.25) (layer "F.Cu") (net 2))
 (segment (start 92.0375 34.4875) (end 91.7 34.15) (width 0.25) (layer "F.Cu") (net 2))
 (segment (start 83.05 46.5625) (end 83.25 46.3625) (width 0.25) (layer "F.Cu") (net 2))
 (segment (start 92.0625 40.3) (end 91.35 40.3) (width 0.25) (layer "F.Cu") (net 2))
 (segment (start 92.0625 37.05) (end 91.7 36.6875) (width 0.25) (layer "F.Cu") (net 2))
 (segment (start 83.25 46.3625) (end 84.4625 45.15) (width 0.25) (layer "F.Cu") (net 2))
 (segment (start 83.05 46.75) (end 83.05 46.5625) (width 0.25) (layer "F.Cu") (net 2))
 (segment (start 92.1 33.75) (end 91.7 34.15) (width 0.25) (layer "F.Cu") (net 2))
 (segment (start 91.7 36.6875) (end 91.7 34.15) (width 0.25) (layer "F.Cu") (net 2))
 (via (at 94.6 41.6) (size 0.8) (drill 0.4) (layers "F.Cu" "B.Cu") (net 2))
 (via (at 92.9 33.75) (size 0.8) (drill 0.4) (layers "F.Cu" "B.Cu") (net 2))
 (via (at 90.75 44.85) (size 0.8) (drill 0.4) (layers "F.Cu" "B.Cu") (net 2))
 (via (at 83.05 46.75) (size 0.8) (drill 0.4) (layers "F.Cu" "B.Cu") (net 2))
 (segment (start 91.95 44.25) (end 91.35 44.25) (width 0.25) (layer "B.Cu") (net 2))
 (segment (start 87.019821 44.630179) (end 85.75 45.9) (width 0.25) (layer "B.Cu") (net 2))
 (segment (start 92.8375 33.6875) (end 92.8375 32.75) (width 0.25) (layer "B.Cu") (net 2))
 (segment (start 94.6 41.6) (end 91.95 44.25) (width 0.25) (layer "B.Cu") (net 2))
 (segment (start 94.6 41.6) (end 94.874614 41.6) (width 0.25) (layer "B.Cu") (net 2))
 (segment (start 94.874614 41.6) (end 96.074614 42.8) (width 0.25) (layer "B.Cu") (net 2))
 (segment (start 91.35 44.25) (end 90.75 44.85) (width 0.25) (layer "B.Cu") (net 2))
 (segment (start 83.05 46.75) (end 81.85 46.75) (width 0.25) (layer "B.Cu") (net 2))
 (segment (start 90.530179 44.630179) (end 87.019821 44.630179) (width 0.25) (layer "B.Cu") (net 2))
 (segment (start 81.85 46.75) (end 81.3 46.2) (width 0.25) (layer "B.Cu") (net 2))
 (segment (start 85.75 45.9) (end 84.9 46.75) (width 0.25) (layer "B.Cu") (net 2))
 (segment (start 84.9 46.75) (end 83.05 46.75) (width 0.25) (layer "B.Cu") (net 2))
 (segment (start 92.9 33.75) (end 92.8375 33.6875) (width 0.25) (layer "B.Cu") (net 2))
 (segment (start 90.75 44.85) (end 90.530179 44.630179) (width 0.25) (layer "B.Cu") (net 2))
 (segment (start 96.074614 42.8) (end 97.2 42.8) (width 0.25) (layer "B.Cu") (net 2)))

